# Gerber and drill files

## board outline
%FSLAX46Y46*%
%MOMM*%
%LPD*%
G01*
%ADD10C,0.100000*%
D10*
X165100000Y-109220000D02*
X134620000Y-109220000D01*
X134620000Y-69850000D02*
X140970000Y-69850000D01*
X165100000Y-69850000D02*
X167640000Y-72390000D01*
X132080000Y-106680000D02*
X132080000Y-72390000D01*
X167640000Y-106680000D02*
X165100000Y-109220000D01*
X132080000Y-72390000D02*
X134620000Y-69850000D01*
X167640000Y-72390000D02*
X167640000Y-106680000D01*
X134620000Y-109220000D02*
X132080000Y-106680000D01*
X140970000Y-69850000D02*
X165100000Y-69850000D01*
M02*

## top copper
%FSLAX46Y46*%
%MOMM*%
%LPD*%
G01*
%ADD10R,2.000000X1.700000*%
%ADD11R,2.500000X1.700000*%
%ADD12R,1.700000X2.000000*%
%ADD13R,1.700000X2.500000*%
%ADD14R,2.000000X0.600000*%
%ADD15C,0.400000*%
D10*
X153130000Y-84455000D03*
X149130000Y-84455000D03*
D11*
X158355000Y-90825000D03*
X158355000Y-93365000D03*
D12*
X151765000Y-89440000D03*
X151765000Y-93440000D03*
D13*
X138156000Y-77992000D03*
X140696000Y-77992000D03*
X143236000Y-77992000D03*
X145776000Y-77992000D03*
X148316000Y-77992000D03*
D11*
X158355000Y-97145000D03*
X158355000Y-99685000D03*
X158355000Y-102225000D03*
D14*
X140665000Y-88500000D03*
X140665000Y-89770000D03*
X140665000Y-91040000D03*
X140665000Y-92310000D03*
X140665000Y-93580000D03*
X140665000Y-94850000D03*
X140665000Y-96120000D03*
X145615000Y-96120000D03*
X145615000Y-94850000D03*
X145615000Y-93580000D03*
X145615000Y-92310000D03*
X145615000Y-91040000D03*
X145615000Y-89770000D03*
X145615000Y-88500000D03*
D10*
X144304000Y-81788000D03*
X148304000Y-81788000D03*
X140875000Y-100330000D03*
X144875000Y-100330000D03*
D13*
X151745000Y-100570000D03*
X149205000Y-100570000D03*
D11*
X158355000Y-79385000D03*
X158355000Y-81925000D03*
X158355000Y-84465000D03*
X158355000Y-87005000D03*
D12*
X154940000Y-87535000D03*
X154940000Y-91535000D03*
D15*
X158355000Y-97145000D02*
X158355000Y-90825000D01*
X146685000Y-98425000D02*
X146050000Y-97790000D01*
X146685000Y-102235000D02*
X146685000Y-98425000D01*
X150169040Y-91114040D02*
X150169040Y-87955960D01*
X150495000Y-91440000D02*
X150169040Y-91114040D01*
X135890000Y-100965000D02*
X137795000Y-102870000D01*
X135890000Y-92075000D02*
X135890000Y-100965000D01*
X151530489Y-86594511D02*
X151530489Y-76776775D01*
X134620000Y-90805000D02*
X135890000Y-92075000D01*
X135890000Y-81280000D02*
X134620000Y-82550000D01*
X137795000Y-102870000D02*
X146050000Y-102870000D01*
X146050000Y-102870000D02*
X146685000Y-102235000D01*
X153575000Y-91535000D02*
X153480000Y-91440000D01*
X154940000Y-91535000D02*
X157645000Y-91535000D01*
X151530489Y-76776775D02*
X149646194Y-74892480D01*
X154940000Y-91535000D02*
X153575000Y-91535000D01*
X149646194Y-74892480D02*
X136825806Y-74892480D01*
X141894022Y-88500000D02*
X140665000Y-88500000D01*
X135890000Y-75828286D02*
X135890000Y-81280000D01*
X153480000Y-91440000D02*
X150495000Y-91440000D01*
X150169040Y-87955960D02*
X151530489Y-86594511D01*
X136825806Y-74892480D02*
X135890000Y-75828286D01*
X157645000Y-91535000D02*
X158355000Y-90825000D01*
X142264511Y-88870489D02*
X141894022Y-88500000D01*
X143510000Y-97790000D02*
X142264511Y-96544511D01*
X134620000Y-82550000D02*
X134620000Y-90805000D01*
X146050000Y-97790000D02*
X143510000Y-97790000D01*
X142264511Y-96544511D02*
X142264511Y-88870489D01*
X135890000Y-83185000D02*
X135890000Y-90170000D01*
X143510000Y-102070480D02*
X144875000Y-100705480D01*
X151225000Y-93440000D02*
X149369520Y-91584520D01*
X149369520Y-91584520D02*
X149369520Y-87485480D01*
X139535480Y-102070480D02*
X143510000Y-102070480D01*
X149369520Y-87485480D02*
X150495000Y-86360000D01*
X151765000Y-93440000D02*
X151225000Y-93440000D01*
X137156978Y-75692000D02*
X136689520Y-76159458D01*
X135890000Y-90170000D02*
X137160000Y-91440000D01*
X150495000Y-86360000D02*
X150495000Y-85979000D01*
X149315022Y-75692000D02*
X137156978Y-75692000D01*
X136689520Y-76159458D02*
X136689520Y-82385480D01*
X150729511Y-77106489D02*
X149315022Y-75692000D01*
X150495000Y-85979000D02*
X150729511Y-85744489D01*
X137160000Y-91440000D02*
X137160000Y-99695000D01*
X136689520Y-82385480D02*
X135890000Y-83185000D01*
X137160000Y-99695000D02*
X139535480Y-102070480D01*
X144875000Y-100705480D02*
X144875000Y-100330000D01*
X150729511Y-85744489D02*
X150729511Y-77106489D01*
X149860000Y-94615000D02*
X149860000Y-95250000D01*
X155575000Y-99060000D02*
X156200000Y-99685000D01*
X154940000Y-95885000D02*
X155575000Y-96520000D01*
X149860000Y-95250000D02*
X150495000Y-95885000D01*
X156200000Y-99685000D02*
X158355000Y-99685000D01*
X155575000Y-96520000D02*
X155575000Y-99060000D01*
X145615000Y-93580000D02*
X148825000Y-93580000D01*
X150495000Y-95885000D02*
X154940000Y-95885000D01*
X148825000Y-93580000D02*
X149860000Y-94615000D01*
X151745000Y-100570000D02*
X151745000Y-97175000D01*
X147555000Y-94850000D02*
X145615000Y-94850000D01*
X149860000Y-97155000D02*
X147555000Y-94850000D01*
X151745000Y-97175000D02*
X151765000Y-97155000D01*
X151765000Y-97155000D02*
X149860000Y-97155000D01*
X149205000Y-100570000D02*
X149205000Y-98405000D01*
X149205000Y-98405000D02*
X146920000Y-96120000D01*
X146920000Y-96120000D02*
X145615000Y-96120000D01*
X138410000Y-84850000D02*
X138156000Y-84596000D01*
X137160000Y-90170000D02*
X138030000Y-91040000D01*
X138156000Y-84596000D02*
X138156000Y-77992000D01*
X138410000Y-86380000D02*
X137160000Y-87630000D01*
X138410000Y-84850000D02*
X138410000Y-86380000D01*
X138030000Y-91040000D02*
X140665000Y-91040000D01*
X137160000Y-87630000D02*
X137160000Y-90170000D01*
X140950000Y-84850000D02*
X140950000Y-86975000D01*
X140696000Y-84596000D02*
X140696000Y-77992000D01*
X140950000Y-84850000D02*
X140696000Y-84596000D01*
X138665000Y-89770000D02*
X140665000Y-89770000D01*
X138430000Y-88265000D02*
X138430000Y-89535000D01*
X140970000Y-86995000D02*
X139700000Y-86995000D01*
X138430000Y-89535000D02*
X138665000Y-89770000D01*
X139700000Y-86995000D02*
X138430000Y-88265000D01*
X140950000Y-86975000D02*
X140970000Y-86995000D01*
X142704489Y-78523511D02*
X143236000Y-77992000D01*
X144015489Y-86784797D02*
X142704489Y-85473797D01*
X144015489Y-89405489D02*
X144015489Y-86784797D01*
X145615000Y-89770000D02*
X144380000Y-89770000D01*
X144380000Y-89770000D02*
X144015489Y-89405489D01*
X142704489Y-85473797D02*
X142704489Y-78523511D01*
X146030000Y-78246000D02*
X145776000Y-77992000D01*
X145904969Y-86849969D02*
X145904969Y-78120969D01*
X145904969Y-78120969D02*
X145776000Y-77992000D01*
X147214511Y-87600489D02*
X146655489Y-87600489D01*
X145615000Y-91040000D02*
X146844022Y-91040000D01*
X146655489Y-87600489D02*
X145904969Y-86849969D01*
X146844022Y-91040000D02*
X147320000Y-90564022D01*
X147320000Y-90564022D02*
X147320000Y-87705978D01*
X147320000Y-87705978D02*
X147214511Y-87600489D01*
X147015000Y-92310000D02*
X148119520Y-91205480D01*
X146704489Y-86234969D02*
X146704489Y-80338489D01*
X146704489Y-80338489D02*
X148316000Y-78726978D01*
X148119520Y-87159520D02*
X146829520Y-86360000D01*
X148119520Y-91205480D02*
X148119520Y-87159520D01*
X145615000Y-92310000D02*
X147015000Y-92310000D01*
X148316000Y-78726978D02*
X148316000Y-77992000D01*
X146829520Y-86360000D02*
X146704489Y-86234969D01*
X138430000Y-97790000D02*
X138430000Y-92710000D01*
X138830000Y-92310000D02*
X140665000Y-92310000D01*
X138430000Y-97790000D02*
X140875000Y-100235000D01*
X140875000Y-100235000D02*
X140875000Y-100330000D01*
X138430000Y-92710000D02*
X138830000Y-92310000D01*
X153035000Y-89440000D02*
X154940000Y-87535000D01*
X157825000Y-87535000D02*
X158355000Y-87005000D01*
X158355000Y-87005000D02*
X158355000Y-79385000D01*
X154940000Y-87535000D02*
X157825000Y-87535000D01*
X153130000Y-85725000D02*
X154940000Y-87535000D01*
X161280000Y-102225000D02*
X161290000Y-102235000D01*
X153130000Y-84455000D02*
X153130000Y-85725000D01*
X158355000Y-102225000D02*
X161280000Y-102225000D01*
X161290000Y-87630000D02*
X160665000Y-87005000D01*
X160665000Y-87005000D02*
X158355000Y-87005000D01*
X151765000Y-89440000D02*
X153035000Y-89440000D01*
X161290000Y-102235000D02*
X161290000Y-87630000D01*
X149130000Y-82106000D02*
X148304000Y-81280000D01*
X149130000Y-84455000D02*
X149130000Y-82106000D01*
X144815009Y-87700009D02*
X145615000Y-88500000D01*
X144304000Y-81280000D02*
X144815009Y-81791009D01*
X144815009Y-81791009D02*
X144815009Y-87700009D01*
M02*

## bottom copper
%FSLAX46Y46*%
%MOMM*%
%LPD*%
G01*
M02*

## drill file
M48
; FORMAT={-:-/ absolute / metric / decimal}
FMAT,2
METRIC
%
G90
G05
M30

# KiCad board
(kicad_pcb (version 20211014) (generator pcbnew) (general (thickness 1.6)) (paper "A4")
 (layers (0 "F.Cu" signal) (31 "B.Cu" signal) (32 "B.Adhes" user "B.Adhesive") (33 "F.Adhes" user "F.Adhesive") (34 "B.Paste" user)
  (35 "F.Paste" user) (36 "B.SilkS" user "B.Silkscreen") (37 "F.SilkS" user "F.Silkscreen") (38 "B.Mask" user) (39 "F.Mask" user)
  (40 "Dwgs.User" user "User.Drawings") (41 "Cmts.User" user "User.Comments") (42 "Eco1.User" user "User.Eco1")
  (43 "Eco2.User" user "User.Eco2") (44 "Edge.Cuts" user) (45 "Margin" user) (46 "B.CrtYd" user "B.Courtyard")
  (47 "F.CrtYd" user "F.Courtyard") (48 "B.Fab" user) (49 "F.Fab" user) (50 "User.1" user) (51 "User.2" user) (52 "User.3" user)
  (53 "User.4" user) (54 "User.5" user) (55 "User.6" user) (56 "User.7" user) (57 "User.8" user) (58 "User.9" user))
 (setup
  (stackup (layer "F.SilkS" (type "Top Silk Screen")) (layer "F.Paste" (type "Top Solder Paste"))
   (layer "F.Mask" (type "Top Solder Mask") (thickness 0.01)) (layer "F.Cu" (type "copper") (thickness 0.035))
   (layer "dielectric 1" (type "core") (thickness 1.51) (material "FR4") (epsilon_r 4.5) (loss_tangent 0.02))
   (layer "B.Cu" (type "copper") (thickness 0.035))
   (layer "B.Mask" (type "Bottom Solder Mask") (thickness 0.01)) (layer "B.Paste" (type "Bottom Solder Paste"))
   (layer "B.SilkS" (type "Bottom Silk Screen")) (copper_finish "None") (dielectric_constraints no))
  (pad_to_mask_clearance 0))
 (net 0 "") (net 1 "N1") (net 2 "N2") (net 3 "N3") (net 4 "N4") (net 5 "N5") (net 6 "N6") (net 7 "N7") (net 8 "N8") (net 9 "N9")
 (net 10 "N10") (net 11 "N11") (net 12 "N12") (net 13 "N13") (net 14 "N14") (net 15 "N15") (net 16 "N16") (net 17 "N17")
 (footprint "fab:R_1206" (layer "F.Cu") (at 151.13 84.455 180)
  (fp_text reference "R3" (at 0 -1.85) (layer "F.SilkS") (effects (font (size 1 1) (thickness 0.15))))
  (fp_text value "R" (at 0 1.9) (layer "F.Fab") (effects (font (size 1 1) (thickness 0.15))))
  (pad "1" smd rect locked (at -2 0 180) (size 2 1.7) (layers "F.Cu" "F.Paste" "F.Mask") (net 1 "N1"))
  (pad "2" smd rect locked (at 2 0 180) (size 2 1.7) (layers "F.Cu" "F.Paste" "F.Mask") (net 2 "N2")))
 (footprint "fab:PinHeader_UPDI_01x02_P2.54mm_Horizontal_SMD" (layer "F.Cu") (at 158.355 90.825)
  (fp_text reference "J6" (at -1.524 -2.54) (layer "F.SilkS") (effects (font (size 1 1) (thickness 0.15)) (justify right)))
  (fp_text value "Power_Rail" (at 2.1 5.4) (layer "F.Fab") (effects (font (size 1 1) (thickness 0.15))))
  (pad "1" smd rect locked (at 0 0) (size 2.5 1.7) (layers "F.Cu" "F.Paste" "F.Mask") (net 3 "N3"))
  (pad "2" smd rect locked (at 0 2.54) (size 2.5 1.7) (layers "F.Cu" "F.Paste" "F.Mask") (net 3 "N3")))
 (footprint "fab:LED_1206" (layer "F.Cu") (at 151.765 91.44 -90)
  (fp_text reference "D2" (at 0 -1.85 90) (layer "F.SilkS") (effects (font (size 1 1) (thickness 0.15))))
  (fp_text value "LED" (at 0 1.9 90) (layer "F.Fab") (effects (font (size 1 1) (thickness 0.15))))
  (pad "1" smd rect locked (at -2 0 270) (size 2 1.7) (layers "F.Cu" "F.Paste" "F.Mask") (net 1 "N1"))
  (pad "2" smd rect locked (at 2 0 270) (size 2 1.7) (layers "F.Cu" "F.Paste" "F.Mask") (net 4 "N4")))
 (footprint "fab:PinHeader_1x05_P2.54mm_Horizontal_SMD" (layer "F.Cu") (at 138.156 77.992 90)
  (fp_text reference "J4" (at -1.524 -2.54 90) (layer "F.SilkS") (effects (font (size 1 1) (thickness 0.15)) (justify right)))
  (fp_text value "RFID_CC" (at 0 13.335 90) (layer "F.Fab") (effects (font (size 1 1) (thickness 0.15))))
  (pad "1" smd rect locked (at 0 0 90) (size 2.5 1.7) (layers "F.Cu" "F.Paste" "F.Mask") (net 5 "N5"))
  (pad "2" smd rect locked (at 0 2.54 90) (size 2.5 1.7) (layers "F.Cu" "F.Paste" "F.Mask") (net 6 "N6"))
  (pad "3" smd rect locked (at 0 5.08 90) (size 2.5 1.7) (layers "F.Cu" "F.Paste" "F.Mask") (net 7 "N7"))
  (pad "4" smd rect locked (at 0 7.62 90) (size 2.5 1.7) (layers "F.Cu" "F.Paste" "F.Mask") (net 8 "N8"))
  (pad "5" smd rect locked (at 0 10.16 90) (size 2.5 1.7) (layers "F.Cu" "F.Paste" "F.Mask") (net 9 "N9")))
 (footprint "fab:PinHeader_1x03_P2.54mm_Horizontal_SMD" (layer "F.Cu") (at 158.355 97.145)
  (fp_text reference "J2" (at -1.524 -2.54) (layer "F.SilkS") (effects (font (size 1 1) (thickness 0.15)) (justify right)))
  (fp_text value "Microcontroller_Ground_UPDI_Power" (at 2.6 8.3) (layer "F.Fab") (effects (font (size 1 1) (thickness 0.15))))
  (pad "1" smd rect locked (at 0 0) (size 2.5 1.7) (layers "F.Cu" "F.Paste" "F.Mask") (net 3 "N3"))
  (pad "2" smd rect locked (at 0 2.54) (size 2.5 1.7) (layers "F.Cu" "F.Paste" "F.Mask") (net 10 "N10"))
  (pad "3" smd rect locked (at 0 5.08) (size 2.5 1.7) (layers "F.Cu" "F.Paste" "F.Mask") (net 1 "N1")))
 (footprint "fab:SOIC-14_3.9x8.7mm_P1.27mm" (layer "F.Cu") (at 143.14 92.31)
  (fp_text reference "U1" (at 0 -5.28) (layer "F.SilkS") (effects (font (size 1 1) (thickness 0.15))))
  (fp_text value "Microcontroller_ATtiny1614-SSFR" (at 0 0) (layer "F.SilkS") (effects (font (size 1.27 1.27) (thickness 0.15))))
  (pad "1" smd rect (at -2.475 -3.81) (size 2 0.6) (layers "F.Cu" "F.Paste" "F.Mask") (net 3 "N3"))
  (pad "2" smd rect (at -2.475 -2.54) (size 2 0.6) (layers "F.Cu" "F.Paste" "F.Mask") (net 6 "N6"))
  (pad "3" smd rect (at -2.475 -1.27) (size 2 0.6) (layers "F.Cu" "F.Paste" "F.Mask") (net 5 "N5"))
  (pad "4" smd rect (at -2.475 0) (size 2 0.6) (layers "F.Cu" "F.Paste" "F.Mask") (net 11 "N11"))
  (pad "5" smd rect (at -2.475 1.27) (size 2 0.6) (layers "F.Cu" "F.Paste" "F.Mask") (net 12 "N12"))
  (pad "6" smd rect (at -2.475 2.54) (size 2 0.6) (layers "F.Cu" "F.Paste" "F.Mask") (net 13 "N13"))
  (pad "7" smd rect (at -2.475 3.81) (size 2 0.6) (layers "F.Cu" "F.Paste" "F.Mask") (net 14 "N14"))
  (pad "8" smd rect (at 2.475 3.81) (size 2 0.6) (layers "F.Cu" "F.Paste" "F.Mask") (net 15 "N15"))
  (pad "9" smd rect (at 2.475 2.54) (size 2 0.6) (layers "F.Cu" "F.Paste" "F.Mask") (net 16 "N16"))
  (pad "10" smd rect (at 2.475 1.27) (size 2 0.6) (layers "F.Cu" "F.Paste" "F.Mask") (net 10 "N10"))
  (pad "11" smd rect (at 2.475 0) (size 2 0.6) (layers "F.Cu" "F.Paste" "F.Mask") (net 9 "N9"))
  (pad "12" smd rect (at 2.475 -1.27) (size 2 0.6) (layers "F.Cu" "F.Paste" "F.Mask") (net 8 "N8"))
  (pad "13" smd rect (at 2.475 -2.54) (size 2 0.6) (layers "F.Cu" "F.Paste" "F.Mask") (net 7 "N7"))
  (pad "14" smd rect (at 2.475 -3.81) (size 2 0.6) (layers "F.Cu" "F.Paste" "F.Mask") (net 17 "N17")))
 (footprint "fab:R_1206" (layer "F.Cu") (at 146.304 81.788)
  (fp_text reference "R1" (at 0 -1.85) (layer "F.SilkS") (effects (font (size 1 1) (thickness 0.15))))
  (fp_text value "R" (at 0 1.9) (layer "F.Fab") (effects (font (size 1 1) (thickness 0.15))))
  (pad "1" smd rect locked (at -2 0) (size 2 1.7) (layers "F.Cu" "F.Paste" "F.Mask") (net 17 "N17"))
  (pad "2" smd rect locked (at 2 0) (size 2 1.7) (layers "F.Cu" "F.Paste" "F.Mask") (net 2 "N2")))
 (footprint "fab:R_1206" (layer "F.Cu") (at 142.875 100.33)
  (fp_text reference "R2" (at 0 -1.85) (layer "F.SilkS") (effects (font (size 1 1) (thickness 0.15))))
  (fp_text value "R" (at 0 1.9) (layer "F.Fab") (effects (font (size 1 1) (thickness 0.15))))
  (pad "1" smd rect locked (at -2 0) (size 2 1.7) (layers "F.Cu" "F.Paste" "F.Mask") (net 11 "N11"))
  (pad "2" smd rect locked (at 2 0) (size 2 1.7) (layers "F.Cu" "F.Paste" "F.Mask") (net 4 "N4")))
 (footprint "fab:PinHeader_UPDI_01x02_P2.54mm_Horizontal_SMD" (layer "F.Cu") (at 151.745 100.57 -90)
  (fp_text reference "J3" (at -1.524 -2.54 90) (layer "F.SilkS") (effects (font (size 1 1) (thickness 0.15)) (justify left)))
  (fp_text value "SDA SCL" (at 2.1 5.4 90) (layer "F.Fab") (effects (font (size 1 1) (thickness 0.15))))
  (pad "1" smd rect locked (at 0 0 270) (size 2.5 1.7) (layers "F.Cu" "F.Paste" "F.Mask") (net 16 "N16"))
  (pad "2" smd rect locked (at 0 2.54 270) (size 2.5 1.7) (layers "F.Cu" "F.Paste" "F.Mask") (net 15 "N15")))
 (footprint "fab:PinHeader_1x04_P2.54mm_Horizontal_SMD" (layer "F.Cu") (at 158.355 79.385)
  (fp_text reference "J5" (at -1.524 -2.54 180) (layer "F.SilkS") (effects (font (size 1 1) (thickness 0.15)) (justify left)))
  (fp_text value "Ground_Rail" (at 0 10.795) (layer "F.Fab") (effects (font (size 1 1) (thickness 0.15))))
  (pad "1" smd rect locked (at 0 0) (size 2.5 1.7) (layers "F.Cu" "F.Paste" "F.Mask") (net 1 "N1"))
  (pad "2" smd rect locked (at 0 2.54) (size 2.5 1.7) (layers "F.Cu" "F.Paste" "F.Mask") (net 1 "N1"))
  (pad "3" smd rect locked (at 0 5.08) (size 2.5 1.7) (layers "F.Cu" "F.Paste" "F.Mask") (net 1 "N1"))
  (pad "4" smd rect locked (at 0 7.62) (size 2.5 1.7) (layers "F.Cu" "F.Paste" "F.Mask") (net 1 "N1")))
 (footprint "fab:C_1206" (layer "F.Cu") (at 154.94 89.535 -90)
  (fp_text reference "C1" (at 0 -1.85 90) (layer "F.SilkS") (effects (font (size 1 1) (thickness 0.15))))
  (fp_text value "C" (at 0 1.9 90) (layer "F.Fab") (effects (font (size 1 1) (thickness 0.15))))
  (pad "1" smd rect locked (at -2 0 270) (size 2 1.7) (layers "F.Cu" "F.Paste" "F.Mask") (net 1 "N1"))
  (pad "2" smd rect locked (at 2 0 270) (size 2 1.7) (layers "F.Cu" "F.Paste" "F.Mask") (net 3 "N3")))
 (gr_line (start 165.1 109.22) (end 134.62 109.22) (layer "Edge.Cuts") (width 0.1))
 (gr_line (start 134.62 69.85) (end 140.97 69.85) (layer "Edge.Cuts") (width 0.1))
 (gr_line (start 165.1 69.85) (end 167.64 72.39) (layer "Edge.Cuts") (width 0.1))
 (gr_line (start 132.08 106.68) (end 132.08 72.39) (layer "Edge.Cuts") (width 0.1))
 (gr_line (start 167.64 106.68) (end 165.1 109.22) (layer "Edge.Cuts") (width 0.1))
 (gr_line (start 132.08 72.39) (end 134.62 69.85) (layer "Edge.Cuts") (width 0.1))
 (gr_line (start 167.64 72.39) (end 167.64 106.68) (layer "Edge.Cuts") (width 0.1))
 (gr_line (start 134.62 109.22) (end 132.08 106.68) (layer "Edge.Cuts") (width 0.1))
 (gr_line (start 140.97 69.85) (end 165.1 69.85) (layer "Edge.Cuts") (width 0.1))
 (segment (start 158.355 97.145) (end 158.355 90.825) (width 0.4) (layer "F.Cu") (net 3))
 (segment (start 146.685 98.425) (end 146.05 97.79) (width 0.4) (layer "F.Cu") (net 3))
 (segment (start 146.685 102.235) (end 146.685 98.425) (width 0.4) (layer "F.Cu") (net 3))
 (segment (start 150.16904 91.11404) (end 150.16904 87.95596) (width 0.4) (layer "F.Cu") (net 3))
 (segment (start 150.495 91.44) (end 150.16904 91.11404) (width 0.4) (layer "F.Cu") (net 3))
 (segment (start 135.89 100.965) (end 137.795 102.87) (width 0.4) (layer "F.Cu") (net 3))
 (segment (start 135.89 92.075) (end 135.89 100.965) (width 0.4) (layer "F.Cu") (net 3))
 (segment (start 151.530489 86.594511) (end 151.530489 76.776775) (width 0.4) (layer "F.Cu") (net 3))
 (segment (start 134.62 90.805) (end 135.89 92.075) (width 0.4) (layer "F.Cu") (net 3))
 (segment (start 135.89 81.28) (end 134.62 82.55) (width 0.4) (layer "F.Cu") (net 3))
 (segment (start 137.795 102.87) (end 146.05 102.87) (width 0.4) (layer "F.Cu") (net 3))
 (segment (start 146.05 102.87) (end 146.685 102.235) (width 0.4) (layer "F.Cu") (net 3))
 (segment (start 153.575 91.535) (end 153.48 91.44) (width 0.4) (layer "F.Cu") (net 3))
 (segment (start 154.94 91.535) (end 157.645 91.535) (width 0.4) (layer "F.Cu") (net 3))
 (segment (start 151.530489 76.776775) (end 149.646194 74.89248) (width 0.4) (layer "F.Cu") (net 3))
 (segment (start 154.94 91.535) (end 153.575 91.535) (width 0.4) (layer "F.Cu") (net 3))
 (segment (start 149.646194 74.89248) (end 136.825806 74.89248) (width 0.4) (layer "F.Cu") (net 3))
 (segment (start 141.894022 88.5) (end 140.665 88.5) (width 0.4) (layer "F.Cu") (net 3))
 (segment (start 135.89 75.828286) (end 135.89 81.28) (width 0.4) (layer "F.Cu") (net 3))
 (segment (start 153.48 91.44) (end 150.495 91.44) (width 0.4) (layer "F.Cu") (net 3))
 (segment (start 150.16904 87.95596) (end 151.530489 86.594511) (width 0.4) (layer "F.Cu") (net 3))
 (segment (start 136.825806 74.89248) (end 135.89 75.828286) (width 0.4) (layer "F.Cu") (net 3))
 (segment (start 157.645 91.535) (end 158.355 90.825) (width 0.4) (layer "F.Cu") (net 3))
 (segment (start 142.264511 88.870489) (end 141.894022 88.5) (width 0.4) (layer "F.Cu") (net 3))
 (segment (start 143.51 97.79) (end 142.264511 96.544511) (width 0.4) (layer "F.Cu") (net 3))
 (segment (start 134.62 82.55) (end 134.62 90.805) (width 0.4) (layer "F.Cu") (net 3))
 (segment (start 146.05 97.79) (end 143.51 97.79) (width 0.4) (layer "F.Cu") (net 3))
 (segment (start 142.264511 96.544511) (end 142.264511 88.870489) (width 0.4) (layer "F.Cu") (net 3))
 (segment (start 135.89 83.185) (end 135.89 90.17) (width 0.4) (layer "F.Cu") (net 4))
 (segment (start 143.51 102.07048) (end 144.875 100.70548) (width 0.4) (layer "F.Cu") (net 4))
 (segment (start 151.225 93.44) (end 149.36952 91.58452) (width 0.4) (layer "F.Cu") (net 4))
 (segment (start 149.36952 91.58452) (end 149.36952 87.48548) (width 0.4) (layer "F.Cu") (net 4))
 (segment (start 139.53548 102.07048) (end 143.51 102.07048) (width 0.4) (layer "F.Cu") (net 4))
 (segment (start 149.36952 87.48548) (end 150.495 86.36) (width 0.4) (layer "F.Cu") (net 4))
 (segment (start 151.765 93.44) (end 151.225 93.44) (width 0.4) (layer "F.Cu") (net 4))
 (segment (start 137.156978 75.692) (end 136.68952 76.159458) (width 0.4) (layer "F.Cu") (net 4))
 (segment (start 135.89 90.17) (end 137.16 91.44) (width 0.4) (layer "F.Cu") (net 4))
 (segment (start 150.495 86.36) (end 150.495 85.979) (width 0.4) (layer "F.Cu") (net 4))
 (segment (start 149.315022 75.692) (end 137.156978 75.692) (width 0.4) (layer "F.Cu") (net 4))
 (segment (start 136.68952 76.159458) (end 136.68952 82.38548) (width 0.4) (layer "F.Cu") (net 4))
 (segment (start 150.729511 77.106489) (end 149.315022 75.692) (width 0.4) (layer "F.Cu") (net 4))
 (segment (start 150.495 85.979) (end 150.729511 85.744489) (width 0.4) (layer "F.Cu") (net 4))
 (segment (start 137.16 91.44) (end 137.16 99.695) (width 0.4) (layer "F.Cu") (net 4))
 (segment (start 136.68952 82.38548) (end 135.89 83.185) (width 0.4) (layer "F.Cu") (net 4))
 (segment (start 137.16 99.695) (end 139.53548 102.07048) (width 0.4) (layer "F.Cu") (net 4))
 (segment (start 144.875 100.70548) (end 144.875 100.33) (width 0.4) (layer "F.Cu") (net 4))
 (segment (start 150.729511 85.744489) (end 150.729511 77.106489) (width 0.4) (layer "F.Cu") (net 4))
 (segment (start 149.86 94.615) (end 149.86 95.25) (width 0.4) (layer "F.Cu") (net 10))
 (segment (start 155.575 99.06) (end 156.2 99.685) (width 0.4) (layer "F.Cu") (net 10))
 (segment (start 154.94 95.885) (end 155.575 96.52) (width 0.4) (layer "F.Cu") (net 10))
 (segment (start 149.86 95.25) (end 150.495 95.885) (width 0.4) (layer "F.Cu") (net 10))
 (segment (start 156.2 99.685) (end 158.355 99.685) (width 0.4) (layer "F.Cu") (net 10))
 (segment (start 155.575 96.52) (end 155.575 99.06) (width 0.4) (layer "F.Cu") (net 10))
 (segment (start 145.615 93.58) (end 148.825 93.58) (width 0.4) (layer "F.Cu") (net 10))
 (segment (start 150.495 95.885) (end 154.94 95.885) (width 0.4) (layer "F.Cu") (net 10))
 (segment (start 148.825 93.58) (end 149.86 94.615) (width 0.4) (layer "F.Cu") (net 10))
 (segment (start 151.745 100.57) (end 151.745 97.175) (width 0.4) (layer "F.Cu") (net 16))
 (segment (start 147.555 94.85) (end 145.615 94.85) (width 0.4) (layer "F.Cu") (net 16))
 (segment (start 149.86 97.155) (end 147.555 94.85) (width 0.4) (layer "F.Cu") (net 16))
 (segment (start 151.745 97.175) (end 151.765 97.155) (width 0.4) (layer "F.Cu") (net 16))
 (segment (start 151.765 97.155) (end 149.86 97.155) (width 0.4) (layer "F.Cu") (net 16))
 (segment (start 149.205 100.57) (end 149.205 98.405) (width 0.4) (layer "F.Cu") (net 15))
 (segment (start 149.205 98.405) (end 146.92 96.12) (width 0.4) (layer "F.Cu") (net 15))
 (segment (start 146.92 96.12) (end 145.615 96.12) (width 0.4) (layer "F.Cu") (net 15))
 (segment (start 138.41 84.85) (end 138.156 84.596) (width 0.4) (layer "F.Cu") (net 5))
 (segment (start 137.16 90.17) (end 138.03 91.04) (width 0.4) (layer "F.Cu") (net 5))
 (segment (start 138.156 84.596) (end 138.156 77.992) (width 0.4) (layer "F.Cu") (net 5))
 (segment (start 138.41 86.38) (end 137.16 87.63) (width 0.4) (layer "F.Cu") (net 5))
 (segment (start 138.41 84.85) (end 138.41 86.38) (width 0.4) (layer "F.Cu") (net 5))
 (segment (start 138.03 91.04) (end 140.665 91.04) (width 0.4) (layer "F.Cu") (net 5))
 (segment (start 137.16 87.63) (end 137.16 90.17) (width 0.4) (layer "F.Cu") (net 5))
 (segment (start 140.95 84.85) (end 140.95 86.975) (width 0.4) (layer "F.Cu") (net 6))
 (segment (start 140.696 84.596) (end 140.696 77.992) (width 0.4) (layer "F.Cu") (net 6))
 (segment (start 140.95 84.85) (end 140.696 84.596) (width 0.4) (layer "F.Cu") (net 6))
 (segment (start 138.665 89.77) (end 140.665 89.77) (width 0.4) (layer "F.Cu") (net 6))
 (segment (start 138.43 88.265) (end 138.43 89.535) (width 0.4) (layer "F.Cu") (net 6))
 (segment (start 140.97 86.995) (end 139.7 86.995) (width 0.4) (layer "F.Cu") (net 6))
 (segment (start 138.43 89.535) (end 138.665 89.77) (width 0.4) (layer "F.Cu") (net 6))
 (segment (start 139.7 86.995) (end 138.43 88.265) (width 0.4) (layer "F.Cu") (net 6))
 (segment (start 140.95 86.975) (end 140.97 86.995) (width 0.4) (layer "F.Cu") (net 6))
 (segment (start 142.704489 78.523511) (end 143.236 77.992) (width 0.4) (layer "F.Cu") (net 7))
 (segment (start 144.015489 86.784797) (end 142.704489 85.473797) (width 0.4) (layer "F.Cu") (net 7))
 (segment (start 144.015489 89.405489) (end 144.015489 86.784797) (width 0.4) (layer "F.Cu") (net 7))
 (segment (start 145.615 89.77) (end 144.38 89.77) (width 0.4) (layer "F.Cu") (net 7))
 (segment (start 144.38 89.77) (end 144.015489 89.405489) (width 0.4) (layer "F.Cu") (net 7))
 (segment (start 142.704489 85.473797) (end 142.704489 78.523511) (width 0.4) (layer "F.Cu") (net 7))
 (segment (start 146.03 78.246) (end 145.776 77.992) (width 0.4) (layer "F.Cu") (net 8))
 (segment (start 145.904969 86.849969) (end 145.904969 78.120969) (width 0.4) (layer "F.Cu") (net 8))
 (segment (start 145.904969 78.120969) (end 145.776 77.992) (width 0.4) (layer "F.Cu") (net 8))
 (segment (start 147.214511 87.600489) (end 146.655489 87.600489) (width 0.4) (layer "F.Cu") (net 8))
 (segment (start 145.615 91.04) (end 146.844022 91.04) (width 0.4) (layer "F.Cu") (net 8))
 (segment (start 146.655489 87.600489) (end 145.904969 86.849969) (width 0.4) (layer "F.Cu") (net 8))
 (segment (start 146.844022 91.04) (end 147.32 90.564022) (width 0.4) (layer "F.Cu") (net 8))
 (segment (start 147.32 90.564022) (end 147.32 87.705978) (width 0.4) (layer "F.Cu") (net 8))
 (segment (start 147.32 87.705978) (end 147.214511 87.600489) (width 0.4) (layer "F.Cu") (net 8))
 (segment (start 147.015 92.31) (end 148.11952 91.20548) (width 0.4) (layer "F.Cu") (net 9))
 (segment (start 146.704489 86.234969) (end 146.704489 80.338489) (width 0.4) (layer "F.Cu") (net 9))
 (segment (start 146.704489 80.338489) (end 148.316 78.726978) (width 0.4) (layer "F.Cu") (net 9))
 (segment (start 148.11952 87.15952) (end 146.82952 86.36) (width 0.4) (layer "F.Cu") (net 9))
 (segment (start 148.11952 91.20548) (end 148.11952 87.15952) (width 0.4) (layer "F.Cu") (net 9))
 (segment (start 145.615 92.31) (end 147.015 92.31) (width 0.4) (layer "F.Cu") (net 9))
 (segment (start 148.316 78.726978) (end 148.316 77.992) (width 0.4) (layer "F.Cu") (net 9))
 (segment (start 146.82952 86.36) (end 146.704489 86.234969) (width 0.4) (layer "F.Cu") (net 9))
 (segment (start 138.43 97.79) (end 138.43 92.71) (width 0.4) (layer "F.Cu") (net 11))
 (segment (start 138.83 92.31) (end 140.665 92.31) (width 0.4) (layer "F.Cu") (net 11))
 (segment (start 138.43 97.79) (end 140.875 100.235) (width 0.4) (layer "F.Cu") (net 11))
 (segment (start 140.875 100.235) (end 140.875 100.33) (width 0.4) (layer "F.Cu") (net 11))
 (segment (start 138.43 92.71) (end 138.83 92.31) (width 0.4) (layer "F.Cu") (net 11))
 (segment (start 153.035 89.44) (end 154.94 87.535) (width 0.4) (layer "F.Cu") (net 1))
 (segment (start 157.825 87.535) (end 158.355 87.005) (width 0.4) (layer "F.Cu") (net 1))
 (segment (start 158.355 87.005) (end 158.355 79.385) (width 0.4) (layer "F.Cu") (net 1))
 (segment (start 154.94 87.535) (end 157.825 87.535) (width 0.4) (layer "F.Cu") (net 1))
 (segment (start 153.13 85.725) (end 154.94 87.535) (width 0.4) (layer "F.Cu") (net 1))
 (segment (start 161.28 102.225) (end 161.29 102.235) (width 0.4) (layer "F.Cu") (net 1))
 (segment (start 153.13 84.455) (end 153.13 85.725) (width 0.4) (layer "F.Cu") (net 1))
 (segment (start 158.355 102.225) (end 161.28 102.225) (width 0.4) (layer "F.Cu") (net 1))
 (segment (start 161.29 87.63) (end 160.665 87.005) (width 0.4) (layer "F.Cu") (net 1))
 (segment (start 160.665 87.005) (end 158.355 87.005) (width 0.4) (layer "F.Cu") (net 1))
 (segment (start 151.765 89.44) (end 153.035 89.44) (width 0.4) (layer "F.Cu") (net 1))
 (segment (start 161.29 102.235) (end 161.29 87.63) (width 0.4) (layer "F.Cu") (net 1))
 (segment (start 149.13 82.106) (end 148.304 81.28) (width 0.4) (layer "F.Cu") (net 2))
 (segment (start 149.13 84.455) (end 149.13 82.106) (width 0.4) (layer "F.Cu") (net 2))
 (segment (start 144.815009 87.700009) (end 145.615 88.5) (width 0.4) (layer "F.Cu") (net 17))
 (segment (start 144.304 81.28) (end 144.815009 81.791009) (width 0.4) (layer "F.Cu") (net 17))
 (segment (start 144.815009 81.791009) (end 144.815009 87.700009) (width 0.4) (layer "F.Cu") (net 17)))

